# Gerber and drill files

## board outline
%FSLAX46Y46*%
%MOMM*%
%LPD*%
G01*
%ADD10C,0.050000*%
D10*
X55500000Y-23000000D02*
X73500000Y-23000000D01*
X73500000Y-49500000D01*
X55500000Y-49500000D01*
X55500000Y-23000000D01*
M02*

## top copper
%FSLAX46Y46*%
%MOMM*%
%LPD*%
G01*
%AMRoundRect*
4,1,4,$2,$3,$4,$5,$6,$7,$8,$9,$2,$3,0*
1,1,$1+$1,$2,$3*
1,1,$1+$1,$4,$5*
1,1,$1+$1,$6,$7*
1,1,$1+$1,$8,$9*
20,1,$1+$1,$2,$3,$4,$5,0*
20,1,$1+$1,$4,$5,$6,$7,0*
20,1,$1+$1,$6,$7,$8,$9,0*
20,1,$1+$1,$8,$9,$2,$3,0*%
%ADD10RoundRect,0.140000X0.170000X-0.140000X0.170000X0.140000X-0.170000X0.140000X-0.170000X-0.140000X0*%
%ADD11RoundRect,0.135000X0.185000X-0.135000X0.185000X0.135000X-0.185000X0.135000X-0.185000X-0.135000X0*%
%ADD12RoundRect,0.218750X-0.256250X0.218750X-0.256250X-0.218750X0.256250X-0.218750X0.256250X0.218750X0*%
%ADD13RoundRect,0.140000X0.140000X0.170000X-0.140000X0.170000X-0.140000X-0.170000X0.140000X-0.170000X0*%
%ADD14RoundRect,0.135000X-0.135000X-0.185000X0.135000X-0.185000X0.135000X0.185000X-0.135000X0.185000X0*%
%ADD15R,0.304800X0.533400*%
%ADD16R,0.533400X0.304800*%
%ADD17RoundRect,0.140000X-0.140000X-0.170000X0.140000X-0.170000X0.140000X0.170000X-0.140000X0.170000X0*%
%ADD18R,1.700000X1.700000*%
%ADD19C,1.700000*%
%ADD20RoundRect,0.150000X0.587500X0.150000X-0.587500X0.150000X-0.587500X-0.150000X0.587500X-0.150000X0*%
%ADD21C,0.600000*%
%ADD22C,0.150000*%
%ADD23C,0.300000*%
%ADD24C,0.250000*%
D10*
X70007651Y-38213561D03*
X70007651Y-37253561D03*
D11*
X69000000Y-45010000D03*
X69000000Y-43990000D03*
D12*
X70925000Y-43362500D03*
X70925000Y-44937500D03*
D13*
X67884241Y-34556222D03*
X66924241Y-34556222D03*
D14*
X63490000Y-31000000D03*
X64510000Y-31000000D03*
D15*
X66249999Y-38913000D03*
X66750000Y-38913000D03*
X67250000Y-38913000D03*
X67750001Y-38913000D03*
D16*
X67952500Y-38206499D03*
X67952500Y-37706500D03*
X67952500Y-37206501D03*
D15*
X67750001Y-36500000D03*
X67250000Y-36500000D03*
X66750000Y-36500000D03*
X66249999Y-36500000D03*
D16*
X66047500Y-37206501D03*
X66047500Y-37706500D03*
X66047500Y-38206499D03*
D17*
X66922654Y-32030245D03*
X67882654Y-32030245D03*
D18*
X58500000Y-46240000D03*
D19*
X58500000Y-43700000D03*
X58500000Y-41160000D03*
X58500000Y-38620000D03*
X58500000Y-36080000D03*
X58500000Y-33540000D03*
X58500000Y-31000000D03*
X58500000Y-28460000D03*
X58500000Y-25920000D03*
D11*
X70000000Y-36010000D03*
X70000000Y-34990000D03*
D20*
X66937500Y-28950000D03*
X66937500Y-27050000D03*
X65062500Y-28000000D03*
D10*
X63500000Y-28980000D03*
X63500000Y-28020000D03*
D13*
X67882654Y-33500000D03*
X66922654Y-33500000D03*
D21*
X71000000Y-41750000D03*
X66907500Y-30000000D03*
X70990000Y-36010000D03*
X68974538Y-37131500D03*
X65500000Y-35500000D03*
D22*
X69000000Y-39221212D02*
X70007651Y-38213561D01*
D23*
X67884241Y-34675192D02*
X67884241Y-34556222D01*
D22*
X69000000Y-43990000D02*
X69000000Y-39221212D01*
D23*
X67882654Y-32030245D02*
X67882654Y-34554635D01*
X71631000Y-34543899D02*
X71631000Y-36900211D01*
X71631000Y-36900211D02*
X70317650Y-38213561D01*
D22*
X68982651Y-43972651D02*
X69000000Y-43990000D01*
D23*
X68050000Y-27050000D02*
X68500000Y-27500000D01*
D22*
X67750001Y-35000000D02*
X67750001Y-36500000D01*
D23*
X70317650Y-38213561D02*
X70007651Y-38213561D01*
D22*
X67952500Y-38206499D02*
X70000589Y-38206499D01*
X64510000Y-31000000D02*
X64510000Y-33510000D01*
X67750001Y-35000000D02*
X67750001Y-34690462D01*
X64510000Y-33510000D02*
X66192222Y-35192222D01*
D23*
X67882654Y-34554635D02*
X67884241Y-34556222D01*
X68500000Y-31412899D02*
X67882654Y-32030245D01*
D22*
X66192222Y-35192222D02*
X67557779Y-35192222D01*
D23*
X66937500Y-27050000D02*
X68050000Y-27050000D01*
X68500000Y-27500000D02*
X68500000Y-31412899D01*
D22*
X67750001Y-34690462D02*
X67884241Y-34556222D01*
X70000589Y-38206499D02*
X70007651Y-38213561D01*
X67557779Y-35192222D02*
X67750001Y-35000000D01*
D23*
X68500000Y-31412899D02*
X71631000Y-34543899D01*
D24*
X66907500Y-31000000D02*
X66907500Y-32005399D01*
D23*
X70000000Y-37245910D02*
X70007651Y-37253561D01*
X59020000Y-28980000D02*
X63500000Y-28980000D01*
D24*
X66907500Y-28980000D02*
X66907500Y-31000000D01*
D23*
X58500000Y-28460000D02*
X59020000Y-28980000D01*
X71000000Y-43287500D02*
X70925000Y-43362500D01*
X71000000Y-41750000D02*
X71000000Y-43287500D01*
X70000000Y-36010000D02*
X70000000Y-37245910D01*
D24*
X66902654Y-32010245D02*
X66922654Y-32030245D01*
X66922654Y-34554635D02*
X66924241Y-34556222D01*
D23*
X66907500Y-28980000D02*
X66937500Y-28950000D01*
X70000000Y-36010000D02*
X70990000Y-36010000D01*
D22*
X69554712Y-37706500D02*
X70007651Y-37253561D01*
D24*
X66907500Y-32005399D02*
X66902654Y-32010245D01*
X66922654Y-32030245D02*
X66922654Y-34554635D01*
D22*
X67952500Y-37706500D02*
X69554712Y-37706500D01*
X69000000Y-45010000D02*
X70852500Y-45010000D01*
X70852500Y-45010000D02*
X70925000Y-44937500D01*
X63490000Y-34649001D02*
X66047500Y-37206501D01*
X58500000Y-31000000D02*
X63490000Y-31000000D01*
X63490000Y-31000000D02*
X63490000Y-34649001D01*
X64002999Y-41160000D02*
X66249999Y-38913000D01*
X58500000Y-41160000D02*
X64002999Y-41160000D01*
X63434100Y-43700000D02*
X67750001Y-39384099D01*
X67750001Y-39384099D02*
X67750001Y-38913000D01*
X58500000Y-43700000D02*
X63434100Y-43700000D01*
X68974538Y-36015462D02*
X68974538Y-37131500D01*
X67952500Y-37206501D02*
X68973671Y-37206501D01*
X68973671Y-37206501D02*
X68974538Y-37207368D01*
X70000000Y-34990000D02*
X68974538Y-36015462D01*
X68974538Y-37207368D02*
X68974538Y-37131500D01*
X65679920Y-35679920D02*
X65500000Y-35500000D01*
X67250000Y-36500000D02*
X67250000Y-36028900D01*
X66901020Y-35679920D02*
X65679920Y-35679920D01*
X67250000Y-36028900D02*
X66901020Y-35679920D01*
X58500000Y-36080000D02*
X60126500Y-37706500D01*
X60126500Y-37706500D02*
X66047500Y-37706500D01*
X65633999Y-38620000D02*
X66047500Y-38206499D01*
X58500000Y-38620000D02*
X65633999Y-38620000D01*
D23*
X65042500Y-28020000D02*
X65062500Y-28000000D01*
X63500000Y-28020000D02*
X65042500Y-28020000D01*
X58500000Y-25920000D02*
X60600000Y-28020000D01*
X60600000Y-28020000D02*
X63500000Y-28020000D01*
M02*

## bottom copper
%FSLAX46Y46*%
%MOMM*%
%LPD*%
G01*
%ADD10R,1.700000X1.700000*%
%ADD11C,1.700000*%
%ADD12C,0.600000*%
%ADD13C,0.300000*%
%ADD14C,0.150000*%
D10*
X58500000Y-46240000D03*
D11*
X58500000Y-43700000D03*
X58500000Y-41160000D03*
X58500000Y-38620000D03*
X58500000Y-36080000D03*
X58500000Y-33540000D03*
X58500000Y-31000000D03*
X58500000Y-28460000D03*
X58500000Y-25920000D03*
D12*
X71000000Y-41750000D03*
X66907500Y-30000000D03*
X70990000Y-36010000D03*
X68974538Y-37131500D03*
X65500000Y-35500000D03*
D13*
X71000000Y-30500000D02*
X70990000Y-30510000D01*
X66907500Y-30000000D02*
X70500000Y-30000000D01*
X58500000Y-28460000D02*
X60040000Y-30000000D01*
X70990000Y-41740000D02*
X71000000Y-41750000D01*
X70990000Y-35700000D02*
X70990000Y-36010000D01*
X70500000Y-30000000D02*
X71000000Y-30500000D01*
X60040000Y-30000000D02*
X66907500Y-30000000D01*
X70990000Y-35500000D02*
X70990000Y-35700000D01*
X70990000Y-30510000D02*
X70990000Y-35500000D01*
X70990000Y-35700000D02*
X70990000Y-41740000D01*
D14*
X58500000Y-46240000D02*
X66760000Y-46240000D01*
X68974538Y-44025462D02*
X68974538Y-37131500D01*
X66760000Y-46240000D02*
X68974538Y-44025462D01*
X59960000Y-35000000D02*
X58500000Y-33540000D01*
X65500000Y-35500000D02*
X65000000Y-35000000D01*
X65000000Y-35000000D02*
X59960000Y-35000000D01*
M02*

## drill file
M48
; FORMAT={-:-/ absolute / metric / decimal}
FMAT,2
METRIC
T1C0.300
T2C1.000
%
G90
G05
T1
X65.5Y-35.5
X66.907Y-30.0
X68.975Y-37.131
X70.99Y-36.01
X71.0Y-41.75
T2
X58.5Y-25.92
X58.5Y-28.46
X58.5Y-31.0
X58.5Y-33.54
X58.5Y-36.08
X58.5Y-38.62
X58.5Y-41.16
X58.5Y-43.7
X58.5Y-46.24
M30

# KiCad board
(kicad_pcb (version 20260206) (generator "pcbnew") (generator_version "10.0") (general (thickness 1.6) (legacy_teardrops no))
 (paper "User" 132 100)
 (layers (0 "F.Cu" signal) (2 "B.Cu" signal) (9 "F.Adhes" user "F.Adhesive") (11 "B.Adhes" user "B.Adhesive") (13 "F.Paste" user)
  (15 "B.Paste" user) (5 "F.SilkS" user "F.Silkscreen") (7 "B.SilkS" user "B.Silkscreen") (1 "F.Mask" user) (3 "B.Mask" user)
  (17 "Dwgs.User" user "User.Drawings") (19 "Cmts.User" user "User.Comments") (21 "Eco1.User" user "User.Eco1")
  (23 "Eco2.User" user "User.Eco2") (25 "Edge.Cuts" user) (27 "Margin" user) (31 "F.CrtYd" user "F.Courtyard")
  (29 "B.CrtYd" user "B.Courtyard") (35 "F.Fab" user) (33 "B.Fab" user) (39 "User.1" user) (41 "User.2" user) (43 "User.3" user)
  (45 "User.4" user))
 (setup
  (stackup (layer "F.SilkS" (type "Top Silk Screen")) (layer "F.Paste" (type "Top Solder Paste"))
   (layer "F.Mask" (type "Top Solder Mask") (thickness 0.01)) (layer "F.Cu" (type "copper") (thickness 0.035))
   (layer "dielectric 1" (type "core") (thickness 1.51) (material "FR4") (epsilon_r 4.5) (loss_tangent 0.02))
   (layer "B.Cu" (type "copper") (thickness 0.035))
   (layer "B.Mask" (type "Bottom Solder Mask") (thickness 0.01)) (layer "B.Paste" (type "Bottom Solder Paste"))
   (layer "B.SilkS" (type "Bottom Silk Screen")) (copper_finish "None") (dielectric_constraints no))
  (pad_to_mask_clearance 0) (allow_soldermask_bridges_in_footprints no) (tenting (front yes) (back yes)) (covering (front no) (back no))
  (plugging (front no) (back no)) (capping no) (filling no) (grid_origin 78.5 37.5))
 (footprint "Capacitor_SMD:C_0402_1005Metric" (layer "F.Cu") (at 70.007651 37.733561 90)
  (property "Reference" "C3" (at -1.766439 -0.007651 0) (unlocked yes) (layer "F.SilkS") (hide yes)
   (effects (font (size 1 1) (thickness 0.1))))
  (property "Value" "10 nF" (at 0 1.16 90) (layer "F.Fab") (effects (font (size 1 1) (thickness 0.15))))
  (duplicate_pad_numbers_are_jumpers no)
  (pad "1" smd roundrect (at -0.48 0 90) (size 0.56 0.62) (layers "F.Cu" "F.Mask" "F.Paste") (roundrect_rratio 0.25) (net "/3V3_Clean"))
  (pad "2" smd roundrect (at 0.48 0 90) (size 0.56 0.62) (layers "F.Cu" "F.Mask" "F.Paste") (roundrect_rratio 0.25) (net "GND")))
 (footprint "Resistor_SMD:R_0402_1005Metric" (layer "F.Cu") (at 69 44.5 90)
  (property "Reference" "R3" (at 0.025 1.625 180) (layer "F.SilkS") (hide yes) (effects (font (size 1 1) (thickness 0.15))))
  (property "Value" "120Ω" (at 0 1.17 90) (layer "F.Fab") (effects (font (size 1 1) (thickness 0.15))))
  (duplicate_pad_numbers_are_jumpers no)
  (pad "1" smd roundrect (at -0.51 0 90) (size 0.54 0.64) (layers "F.Cu" "F.Mask" "F.Paste") (roundrect_rratio 0.25) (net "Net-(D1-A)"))
  (pad "2" smd roundrect (at 0.51 0 90) (size 0.54 0.64) (layers "F.Cu" "F.Mask" "F.Paste") (roundrect_rratio 0.25) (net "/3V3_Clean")))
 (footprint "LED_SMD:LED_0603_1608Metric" (layer "F.Cu") (at 70.925 44.15 -90)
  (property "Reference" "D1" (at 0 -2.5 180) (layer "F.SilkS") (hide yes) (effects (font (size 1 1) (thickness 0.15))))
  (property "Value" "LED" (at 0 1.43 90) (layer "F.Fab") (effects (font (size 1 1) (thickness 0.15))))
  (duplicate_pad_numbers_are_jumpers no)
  (pad "1" smd roundrect (at -0.7875 0 270) (size 0.875 0.95) (layers "F.Cu" "F.Mask" "F.Paste") (roundrect_rratio 0.25) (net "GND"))
  (pad "2" smd roundrect (at 0.7875 0 270) (size 0.875 0.95) (layers "F.Cu" "F.Mask" "F.Paste") (roundrect_rratio 0.25) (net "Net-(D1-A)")))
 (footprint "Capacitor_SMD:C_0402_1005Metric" (layer "F.Cu") (at 67.404241 34.556222 180)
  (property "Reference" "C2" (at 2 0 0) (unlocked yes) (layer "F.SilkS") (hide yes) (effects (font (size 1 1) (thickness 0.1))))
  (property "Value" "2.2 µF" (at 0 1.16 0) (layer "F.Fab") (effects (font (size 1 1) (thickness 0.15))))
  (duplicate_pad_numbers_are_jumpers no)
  (pad "1" smd roundrect (at -0.48 0 180) (size 0.56 0.62) (layers "F.Cu" "F.Mask" "F.Paste") (roundrect_rratio 0.25) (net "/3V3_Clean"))
  (pad "2" smd roundrect (at 0.48 0 180) (size 0.56 0.62) (layers "F.Cu" "F.Mask" "F.Paste") (roundrect_rratio 0.25) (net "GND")))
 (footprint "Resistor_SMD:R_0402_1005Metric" (layer "F.Cu") (at 64 31)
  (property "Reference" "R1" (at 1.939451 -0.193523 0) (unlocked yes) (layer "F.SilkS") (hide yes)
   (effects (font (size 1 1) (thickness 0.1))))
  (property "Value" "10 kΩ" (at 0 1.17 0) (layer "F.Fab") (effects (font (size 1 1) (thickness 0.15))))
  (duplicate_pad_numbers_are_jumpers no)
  (pad "1" smd roundrect (at -0.51 0) (size 0.54 0.64) (layers "F.Cu" "F.Mask" "F.Paste") (roundrect_rratio 0.25) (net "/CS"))
  (pad "2" smd roundrect (at 0.51 0) (size 0.54 0.64) (layers "F.Cu" "F.Mask" "F.Paste") (roundrect_rratio 0.25) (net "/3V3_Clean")))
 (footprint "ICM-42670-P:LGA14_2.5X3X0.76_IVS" (layer "F.Cu") (at 67 37.7065 90)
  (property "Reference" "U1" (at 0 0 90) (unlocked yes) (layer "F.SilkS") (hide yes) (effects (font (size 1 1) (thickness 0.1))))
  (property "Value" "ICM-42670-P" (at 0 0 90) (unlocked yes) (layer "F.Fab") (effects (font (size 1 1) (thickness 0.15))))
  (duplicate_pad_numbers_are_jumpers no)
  (pad "1" smd rect (at -1.2065 -0.750001 180) (size 0.3048 0.5334) (layers "F.Cu" "F.Mask" "F.Paste") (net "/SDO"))
  (pad "2" smd rect (at -1.2065 -0.25 180) (size 0.3048 0.5334) (layers "F.Cu" "F.Mask" "F.Paste") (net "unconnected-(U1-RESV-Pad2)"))
  (pad "3" smd rect (at -1.2065 0.25 180) (size 0.3048 0.5334) (layers "F.Cu" "F.Mask" "F.Paste") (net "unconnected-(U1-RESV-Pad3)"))
  (pad "4" smd rect (at -1.2065 0.750001 180) (size 0.3048 0.5334) (layers "F.Cu" "F.Mask" "F.Paste") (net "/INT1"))
  (pad "5" smd rect (at -0.499999 0.9525 90) (size 0.3048 0.5334) (layers "F.Cu" "F.Mask" "F.Paste") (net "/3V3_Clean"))
  (pad "6" smd rect (at 0 0.9525 90) (size 0.3048 0.5334) (layers "F.Cu" "F.Mask" "F.Paste") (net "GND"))
  (pad "7" smd rect (at 0.499999 0.9525 90) (size 0.3048 0.5334) (layers "F.Cu" "F.Mask" "F.Paste") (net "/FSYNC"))
  (pad "8" smd rect (at 1.2065 0.750001 180) (size 0.3048 0.5334) (layers "F.Cu" "F.Mask" "F.Paste") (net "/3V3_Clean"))
  (pad "9" smd rect (at 1.2065 0.25 180) (size 0.3048 0.5334) (layers "F.Cu" "F.Mask" "F.Paste") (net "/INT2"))
  (pad "10" smd rect (at 1.2065 -0.25 180) (size 0.3048 0.5334) (layers "F.Cu" "F.Mask" "F.Paste") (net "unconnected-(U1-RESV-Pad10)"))
  (pad "11" smd rect (at 1.2065 -0.750001 180) (size 0.3048 0.5334) (layers "F.Cu" "F.Mask" "F.Paste") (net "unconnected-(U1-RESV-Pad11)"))
  (pad "12" smd rect (at 0.499999 -0.9525 90) (size 0.3048 0.5334) (layers "F.Cu" "F.Mask" "F.Paste") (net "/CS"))
  (pad "13" smd rect (at 0 -0.9525 90) (size 0.3048 0.5334) (layers "F.Cu" "F.Mask" "F.Paste") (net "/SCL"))
  (pad "14" smd rect (at -0.499999 -0.9525 90) (size 0.3048 0.5334) (layers "F.Cu" "F.Mask" "F.Paste") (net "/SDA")))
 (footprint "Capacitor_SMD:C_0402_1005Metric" (layer "F.Cu") (at 67.402654 32.030245)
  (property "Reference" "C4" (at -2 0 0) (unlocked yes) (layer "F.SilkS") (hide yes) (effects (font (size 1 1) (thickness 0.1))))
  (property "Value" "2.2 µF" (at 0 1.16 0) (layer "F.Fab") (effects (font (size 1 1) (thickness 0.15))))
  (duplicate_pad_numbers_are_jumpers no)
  (pad "1" smd roundrect (at -0.48 0) (size 0.56 0.62) (layers "F.Cu" "F.Mask" "F.Paste") (roundrect_rratio 0.25) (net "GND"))
  (pad "2" smd roundrect (at 0.48 0) (size 0.56 0.62) (layers "F.Cu" "F.Mask" "F.Paste") (roundrect_rratio 0.25) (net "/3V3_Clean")))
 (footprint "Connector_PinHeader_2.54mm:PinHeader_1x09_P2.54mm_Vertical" (layer "F.Cu") (at 58.5 46.24 180)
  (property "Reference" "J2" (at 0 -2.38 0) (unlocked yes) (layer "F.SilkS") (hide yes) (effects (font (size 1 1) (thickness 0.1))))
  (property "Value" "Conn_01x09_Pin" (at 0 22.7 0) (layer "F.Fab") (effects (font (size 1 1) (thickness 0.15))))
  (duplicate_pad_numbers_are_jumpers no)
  (pad "1" thru_hole rect (at 0 0 180) (size 1.7 1.7) (drill 1) (layers "*.Cu" "*.Mask") (remove_unused_layers no) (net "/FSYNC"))
  (pad "2" thru_hole circle (at 0 2.54 180) (size 1.7 1.7) (drill 1) (layers "*.Cu" "*.Mask") (remove_unused_layers no) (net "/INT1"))
  (pad "3" thru_hole circle (at 0 5.08 180) (size 1.7 1.7) (drill 1) (layers "*.Cu" "*.Mask") (remove_unused_layers no) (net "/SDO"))
  (pad "4" thru_hole circle (at 0 7.62 180) (size 1.7 1.7) (drill 1) (layers "*.Cu" "*.Mask") (remove_unused_layers no) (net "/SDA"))
  (pad "5" thru_hole circle (at 0 10.16 180) (size 1.7 1.7) (drill 1) (layers "*.Cu" "*.Mask") (remove_unused_layers no) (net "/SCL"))
  (pad "6" thru_hole circle (at 0 12.7 180) (size 1.7 1.7) (drill 1) (layers "*.Cu" "*.Mask") (remove_unused_layers no) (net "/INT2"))
  (pad "7" thru_hole circle (at 0 15.24 180) (size 1.7 1.7) (drill 1) (layers "*.Cu" "*.Mask") (remove_unused_layers no) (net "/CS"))
  (pad "8" thru_hole circle (at 0 17.78 180) (size 1.7 1.7) (drill 1) (layers "*.Cu" "*.Mask") (remove_unused_layers no) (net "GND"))
  (pad "9" thru_hole circle (at 0 20.32 180) (size 1.7 1.7) (drill 1) (layers "*.Cu" "*.Mask") (remove_unused_layers no)
   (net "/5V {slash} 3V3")))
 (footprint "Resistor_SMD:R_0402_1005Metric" (layer "F.Cu") (at 70 35.5 90)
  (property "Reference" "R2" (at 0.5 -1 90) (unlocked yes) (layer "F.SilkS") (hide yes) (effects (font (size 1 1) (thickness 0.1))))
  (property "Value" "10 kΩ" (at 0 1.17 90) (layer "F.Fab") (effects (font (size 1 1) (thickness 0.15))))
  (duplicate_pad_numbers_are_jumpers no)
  (pad "1" smd roundrect (at -0.51 0 90) (size 0.54 0.64) (layers "F.Cu" "F.Mask" "F.Paste") (roundrect_rratio 0.25) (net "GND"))
  (pad "2" smd roundrect (at 0.51 0 90) (size 0.54 0.64) (layers "F.Cu" "F.Mask" "F.Paste") (roundrect_rratio 0.25) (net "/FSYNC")))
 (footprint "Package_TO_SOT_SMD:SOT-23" (layer "F.Cu") (at 66 28 180)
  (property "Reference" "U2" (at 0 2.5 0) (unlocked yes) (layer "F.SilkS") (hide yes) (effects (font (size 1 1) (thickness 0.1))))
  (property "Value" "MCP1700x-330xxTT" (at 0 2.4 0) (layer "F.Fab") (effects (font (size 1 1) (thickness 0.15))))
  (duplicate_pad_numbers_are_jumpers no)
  (pad "1" smd roundrect (at -0.9375 -0.95 180) (size 1.475 0.6) (layers "F.Cu" "F.Mask" "F.Paste") (roundrect_rratio 0.25) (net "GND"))
  (pad "2" smd roundrect (at -0.9375 0.95 180) (size 1.475 0.6) (layers "F.Cu" "F.Mask" "F.Paste") (roundrect_rratio 0.25)
   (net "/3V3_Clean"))
  (pad "3" smd roundrect (at 0.9375 0 180) (size 1.475 0.6) (layers "F.Cu" "F.Mask" "F.Paste") (roundrect_rratio 0.25)
   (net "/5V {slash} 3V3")))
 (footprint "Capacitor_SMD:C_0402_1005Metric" (layer "F.Cu") (at 63.5 28.5 90)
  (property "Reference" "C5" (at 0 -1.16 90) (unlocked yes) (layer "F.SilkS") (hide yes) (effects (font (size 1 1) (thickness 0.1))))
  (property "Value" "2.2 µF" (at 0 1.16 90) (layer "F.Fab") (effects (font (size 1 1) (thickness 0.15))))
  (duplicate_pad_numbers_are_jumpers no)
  (pad "1" smd roundrect (at -0.48 0 90) (size 0.56 0.62) (layers "F.Cu" "F.Mask" "F.Paste") (roundrect_rratio 0.25) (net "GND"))
  (pad "2" smd roundrect (at 0.48 0 90) (size 0.56 0.62) (layers "F.Cu" "F.Mask" "F.Paste") (roundrect_rratio 0.25) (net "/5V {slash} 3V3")))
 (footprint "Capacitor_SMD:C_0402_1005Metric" (layer "F.Cu") (at 67.402654 33.5 180)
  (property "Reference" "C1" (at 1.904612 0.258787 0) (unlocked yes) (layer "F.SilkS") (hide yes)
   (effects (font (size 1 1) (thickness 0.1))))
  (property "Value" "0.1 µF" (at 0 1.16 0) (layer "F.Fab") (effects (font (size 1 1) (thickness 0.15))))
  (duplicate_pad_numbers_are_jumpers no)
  (pad "1" smd roundrect (at -0.48 0 180) (size 0.56 0.62) (layers "F.Cu" "F.Mask" "F.Paste") (roundrect_rratio 0.25) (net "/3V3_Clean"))
  (pad "2" smd roundrect (at 0.48 0 180) (size 0.56 0.62) (layers "F.Cu" "F.Mask" "F.Paste") (roundrect_rratio 0.25) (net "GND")))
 (gr_rect (start 55.5 23) (end 73.5 49.5) (stroke (width 0.05) (type solid)) (fill no) (layer "Edge.Cuts"))
 (segment (start 69 39.221212) (end 70.007651 38.213561) (width 0.15) (layer "F.Cu") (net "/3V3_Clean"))
 (segment (start 67.884241 34.675192) (end 67.884241 34.556222) (width 0.3) (layer "F.Cu") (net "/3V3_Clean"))
 (segment (start 69 43.99) (end 69 39.221212) (width 0.15) (layer "F.Cu") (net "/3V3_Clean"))
 (segment (start 67.882654 32.030245) (end 67.882654 34.554635) (width 0.3) (layer "F.Cu") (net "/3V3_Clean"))
 (segment (start 71.631 34.543899) (end 71.631 36.900211) (width 0.3) (layer "F.Cu") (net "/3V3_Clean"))
 (segment (start 71.631 36.900211) (end 70.31765 38.213561) (width 0.3) (layer "F.Cu") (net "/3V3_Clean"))
 (segment (start 68.982651 43.972651) (end 69 43.99) (width 0.15) (layer "F.Cu") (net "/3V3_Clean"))
 (segment (start 68.05 27.05) (end 68.5 27.5) (width 0.3) (layer "F.Cu") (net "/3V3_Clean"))
 (segment (start 67.750001 35) (end 67.750001 36.5) (width 0.15) (layer "F.Cu") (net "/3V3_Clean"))
 (segment (start 70.31765 38.213561) (end 70.007651 38.213561) (width 0.3) (layer "F.Cu") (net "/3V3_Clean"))
 (segment (start 67.9525 38.206499) (end 70.000589 38.206499) (width 0.15) (layer "F.Cu") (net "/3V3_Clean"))
 (segment (start 64.51 31) (end 64.51 33.51) (width 0.15) (layer "F.Cu") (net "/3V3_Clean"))
 (segment (start 67.750001 35) (end 67.750001 34.690462) (width 0.15) (layer "F.Cu") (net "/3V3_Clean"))
 (segment (start 64.51 33.51) (end 66.192222 35.192222) (width 0.15) (layer "F.Cu") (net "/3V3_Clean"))
 (segment (start 67.882654 34.554635) (end 67.884241 34.556222) (width 0.3) (layer "F.Cu") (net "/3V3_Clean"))
 (segment (start 68.5 31.412899) (end 67.882654 32.030245) (width 0.3) (layer "F.Cu") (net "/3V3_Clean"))
 (segment (start 66.192222 35.192222) (end 67.557779 35.192222) (width 0.15) (layer "F.Cu") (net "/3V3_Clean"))
 (segment (start 66.9375 27.05) (end 68.05 27.05) (width 0.3) (layer "F.Cu") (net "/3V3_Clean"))
 (segment (start 68.5 27.5) (end 68.5 31.412899) (width 0.3) (layer "F.Cu") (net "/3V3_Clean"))
 (segment (start 67.750001 34.690462) (end 67.884241 34.556222) (width 0.15) (layer "F.Cu") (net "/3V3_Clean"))
 (segment (start 70.000589 38.206499) (end 70.007651 38.213561) (width 0.15) (layer "F.Cu") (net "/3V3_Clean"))
 (segment (start 67.557779 35.192222) (end 67.750001 35) (width 0.15) (layer "F.Cu") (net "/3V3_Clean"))
 (segment (start 68.5 31.412899) (end 71.631 34.543899) (width 0.3) (layer "F.Cu") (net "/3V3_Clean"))
 (segment (start 66.9075 31) (end 66.9075 32.005399) (width 0.25) (layer "F.Cu") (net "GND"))
 (segment (start 70 37.24591) (end 70.007651 37.253561) (width 0.3) (layer "F.Cu") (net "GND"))
 (segment (start 59.02 28.98) (end 63.5 28.98) (width 0.3) (layer "F.Cu") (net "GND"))
 (segment (start 66.9075 28.98) (end 66.9075 31) (width 0.25) (layer "F.Cu") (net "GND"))
 (segment (start 58.5 28.46) (end 59.02 28.98) (width 0.3) (layer "F.Cu") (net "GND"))
 (segment (start 71 43.2875) (end 70.925 43.3625) (width 0.3) (layer "F.Cu") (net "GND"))
 (segment (start 71 41.75) (end 71 43.2875) (width 0.3) (layer "F.Cu") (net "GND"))
 (segment (start 70 36.01) (end 70 37.24591) (width 0.3) (layer "F.Cu") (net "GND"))
 (segment (start 66.902654 32.010245) (end 66.922654 32.030245) (width 0.25) (layer "F.Cu") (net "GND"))
 (segment (start 66.922654 34.554635) (end 66.924241 34.556222) (width 0.25) (layer "F.Cu") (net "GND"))
 (segment (start 66.9075 28.98) (end 66.9375 28.95) (width 0.3) (layer "F.Cu") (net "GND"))
 (segment (start 70 36.01) (end 70.99 36.01) (width 0.3) (layer "F.Cu") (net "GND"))
 (segment (start 69.554712 37.7065) (end 70.007651 37.253561) (width 0.15) (layer "F.Cu") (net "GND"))
 (segment (start 66.9075 32.005399) (end 66.902654 32.010245) (width 0.25) (layer "F.Cu") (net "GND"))
 (segment (start 66.922654 32.030245) (end 66.922654 34.554635) (width 0.25) (layer "F.Cu") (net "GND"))
 (segment (start 67.9525 37.7065) (end 69.554712 37.7065) (width 0.15) (layer "F.Cu") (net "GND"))
 (via (at 71 41.75) (size 0.6) (drill 0.3) (layers "F.Cu" "B.Cu") (capping no) (covering (front no) (back no))
  (plugging (front no) (back no)) (filling no) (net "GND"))
 (via (at 66.9075 30) (size 0.6) (drill 0.3) (layers "F.Cu" "B.Cu") (capping no) (covering (front no) (back no))
  (plugging (front no) (back no)) (filling no) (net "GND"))
 (via (at 70.99 36.01) (size 0.6) (drill 0.3) (layers "F.Cu" "B.Cu") (capping no) (covering (front no) (back no))
  (plugging (front no) (back no)) (filling no) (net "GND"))
 (segment (start 71 30.5) (end 70.99 30.51) (width 0.3) (layer "B.Cu") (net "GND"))
 (segment (start 66.9075 30) (end 70.5 30) (width 0.3) (layer "B.Cu") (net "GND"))
 (segment (start 58.5 28.46) (end 60.04 30) (width 0.3) (layer "B.Cu") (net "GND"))
 (segment (start 70.99 41.74) (end 71 41.75) (width 0.3) (layer "B.Cu") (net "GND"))
 (segment (start 70.99 35.7) (end 70.99 36.01) (width 0.3) (layer "B.Cu") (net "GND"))
 (segment (start 70.5 30) (end 71 30.5) (width 0.3) (layer "B.Cu") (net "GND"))
 (segment (start 60.04 30) (end 66.9075 30) (width 0.3) (layer "B.Cu") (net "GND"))
 (segment (start 70.99 35.5) (end 70.99 35.7) (width 0.3) (layer "B.Cu") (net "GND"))
 (segment (start 70.99 30.51) (end 70.99 35.5) (width 0.3) (layer "B.Cu") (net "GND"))
 (segment (start 70.99 35.7) (end 70.99 41.74) (width 0.3) (layer "B.Cu") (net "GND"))
 (segment (start 69 45.01) (end 70.8525 45.01) (width 0.15) (layer "F.Cu") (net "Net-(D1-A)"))
 (segment (start 70.8525 45.01) (end 70.925 44.9375) (width 0.15) (layer "F.Cu") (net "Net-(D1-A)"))
 (segment (start 63.49 34.649001) (end 66.0475 37.206501) (width 0.15) (layer "F.Cu") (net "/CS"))
 (segment (start 58.5 31) (end 63.49 31) (width 0.15) (layer "F.Cu") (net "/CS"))
 (segment (start 63.49 31) (end 63.49 34.649001) (width 0.15) (layer "F.Cu") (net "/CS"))
 (segment (start 64.002999 41.16) (end 66.249999 38.913) (width 0.15) (layer "F.Cu") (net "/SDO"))
 (segment (start 58.5 41.16) (end 64.002999 41.16) (width 0.15) (layer "F.Cu") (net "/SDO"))
 (segment (start 63.4341 43.7) (end 67.750001 39.384099) (width 0.15) (layer "F.Cu") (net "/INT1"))
 (segment (start 67.750001 39.384099) (end 67.750001 38.913) (width 0.15) (layer "F.Cu") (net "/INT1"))
 (segment (start 58.5 43.7) (end 63.4341 43.7) (width 0.15) (layer "F.Cu") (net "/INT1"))
 (segment (start 68.974538 36.015462) (end 68.974538 37.1315) (width 0.15) (layer "F.Cu") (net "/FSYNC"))
 (segment (start 67.9525 37.206501) (end 68.973671 37.206501) (width 0.15) (layer "F.Cu") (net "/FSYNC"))
 (segment (start 68.973671 37.206501) (end 68.974538 37.207368) (width 0.15) (layer "F.Cu") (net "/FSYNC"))
 (segment (start 70 34.99) (end 68.974538 36.015462) (width 0.15) (layer "F.Cu") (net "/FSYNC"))
 (segment (start 68.974538 37.207368) (end 68.974538 37.1315) (width 0.15) (layer "F.Cu") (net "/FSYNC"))
 (via (at 68.974538 37.1315) (size 0.6) (drill 0.3) (layers "F.Cu" "B.Cu") (capping no) (covering (front no) (back no))
  (plugging (front no) (back no)) (filling no) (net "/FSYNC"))
 (segment (start 58.5 46.24) (end 66.76 46.24) (width 0.15) (layer "B.Cu") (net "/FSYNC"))
 (segment (start 68.974538 44.025462) (end 68.974538 37.1315) (width 0.15) (layer "B.Cu") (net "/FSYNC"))
 (segment (start 66.76 46.24) (end 68.974538 44.025462) (width 0.15) (layer "B.Cu") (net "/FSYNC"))
 (segment (start 65.67992 35.67992) (end 65.5 35.5) (width 0.15) (layer "F.Cu") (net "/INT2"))
 (segment (start 67.25 36.5) (end 67.25 36.0289) (width 0.15) (layer "F.Cu") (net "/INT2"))
 (segment (start 66.90102 35.67992) (end 65.67992 35.67992) (width 0.15) (layer "F.Cu") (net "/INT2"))
 (segment (start 67.25 36.0289) (end 66.90102 35.67992) (width 0.15) (layer "F.Cu") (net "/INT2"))
 (via (at 65.5 35.5) (size 0.6) (drill 0.3) (layers "F.Cu" "B.Cu") (capping no) (covering (front no) (back no))
  (plugging (front no) (back no)) (filling no) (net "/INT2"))
 (segment (start 59.96 35) (end 58.5 33.54) (width 0.15) (layer "B.Cu") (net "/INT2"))
 (segment (start 65.5 35.5) (end 65 35) (width 0.15) (layer "B.Cu") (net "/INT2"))
 (segment (start 65 35) (end 59.96 35) (width 0.15) (layer "B.Cu") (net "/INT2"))
 (segment (start 58.5 36.08) (end 60.1265 37.7065) (width 0.15) (layer "F.Cu") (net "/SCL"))
 (segment (start 60.1265 37.7065) (end 66.0475 37.7065) (width 0.15) (layer "F.Cu") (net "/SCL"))
 (segment (start 65.633999 38.62) (end 66.0475 38.206499) (width 0.15) (layer "F.Cu") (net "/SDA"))
 (segment (start 58.5 38.62) (end 65.633999 38.62) (width 0.15) (layer "F.Cu") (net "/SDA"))
 (segment (start 65.0425 28.02) (end 65.0625 28) (width 0.3) (layer "F.Cu") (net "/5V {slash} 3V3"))
 (segment (start 63.5 28.02) (end 65.0425 28.02) (width 0.3) (layer "F.Cu") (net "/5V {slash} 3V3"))
 (segment (start 58.5 25.92) (end 60.6 28.02) (width 0.3) (layer "F.Cu") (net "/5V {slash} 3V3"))
 (segment (start 60.6 28.02) (end 63.5 28.02) (width 0.3) (layer "F.Cu") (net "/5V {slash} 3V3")))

